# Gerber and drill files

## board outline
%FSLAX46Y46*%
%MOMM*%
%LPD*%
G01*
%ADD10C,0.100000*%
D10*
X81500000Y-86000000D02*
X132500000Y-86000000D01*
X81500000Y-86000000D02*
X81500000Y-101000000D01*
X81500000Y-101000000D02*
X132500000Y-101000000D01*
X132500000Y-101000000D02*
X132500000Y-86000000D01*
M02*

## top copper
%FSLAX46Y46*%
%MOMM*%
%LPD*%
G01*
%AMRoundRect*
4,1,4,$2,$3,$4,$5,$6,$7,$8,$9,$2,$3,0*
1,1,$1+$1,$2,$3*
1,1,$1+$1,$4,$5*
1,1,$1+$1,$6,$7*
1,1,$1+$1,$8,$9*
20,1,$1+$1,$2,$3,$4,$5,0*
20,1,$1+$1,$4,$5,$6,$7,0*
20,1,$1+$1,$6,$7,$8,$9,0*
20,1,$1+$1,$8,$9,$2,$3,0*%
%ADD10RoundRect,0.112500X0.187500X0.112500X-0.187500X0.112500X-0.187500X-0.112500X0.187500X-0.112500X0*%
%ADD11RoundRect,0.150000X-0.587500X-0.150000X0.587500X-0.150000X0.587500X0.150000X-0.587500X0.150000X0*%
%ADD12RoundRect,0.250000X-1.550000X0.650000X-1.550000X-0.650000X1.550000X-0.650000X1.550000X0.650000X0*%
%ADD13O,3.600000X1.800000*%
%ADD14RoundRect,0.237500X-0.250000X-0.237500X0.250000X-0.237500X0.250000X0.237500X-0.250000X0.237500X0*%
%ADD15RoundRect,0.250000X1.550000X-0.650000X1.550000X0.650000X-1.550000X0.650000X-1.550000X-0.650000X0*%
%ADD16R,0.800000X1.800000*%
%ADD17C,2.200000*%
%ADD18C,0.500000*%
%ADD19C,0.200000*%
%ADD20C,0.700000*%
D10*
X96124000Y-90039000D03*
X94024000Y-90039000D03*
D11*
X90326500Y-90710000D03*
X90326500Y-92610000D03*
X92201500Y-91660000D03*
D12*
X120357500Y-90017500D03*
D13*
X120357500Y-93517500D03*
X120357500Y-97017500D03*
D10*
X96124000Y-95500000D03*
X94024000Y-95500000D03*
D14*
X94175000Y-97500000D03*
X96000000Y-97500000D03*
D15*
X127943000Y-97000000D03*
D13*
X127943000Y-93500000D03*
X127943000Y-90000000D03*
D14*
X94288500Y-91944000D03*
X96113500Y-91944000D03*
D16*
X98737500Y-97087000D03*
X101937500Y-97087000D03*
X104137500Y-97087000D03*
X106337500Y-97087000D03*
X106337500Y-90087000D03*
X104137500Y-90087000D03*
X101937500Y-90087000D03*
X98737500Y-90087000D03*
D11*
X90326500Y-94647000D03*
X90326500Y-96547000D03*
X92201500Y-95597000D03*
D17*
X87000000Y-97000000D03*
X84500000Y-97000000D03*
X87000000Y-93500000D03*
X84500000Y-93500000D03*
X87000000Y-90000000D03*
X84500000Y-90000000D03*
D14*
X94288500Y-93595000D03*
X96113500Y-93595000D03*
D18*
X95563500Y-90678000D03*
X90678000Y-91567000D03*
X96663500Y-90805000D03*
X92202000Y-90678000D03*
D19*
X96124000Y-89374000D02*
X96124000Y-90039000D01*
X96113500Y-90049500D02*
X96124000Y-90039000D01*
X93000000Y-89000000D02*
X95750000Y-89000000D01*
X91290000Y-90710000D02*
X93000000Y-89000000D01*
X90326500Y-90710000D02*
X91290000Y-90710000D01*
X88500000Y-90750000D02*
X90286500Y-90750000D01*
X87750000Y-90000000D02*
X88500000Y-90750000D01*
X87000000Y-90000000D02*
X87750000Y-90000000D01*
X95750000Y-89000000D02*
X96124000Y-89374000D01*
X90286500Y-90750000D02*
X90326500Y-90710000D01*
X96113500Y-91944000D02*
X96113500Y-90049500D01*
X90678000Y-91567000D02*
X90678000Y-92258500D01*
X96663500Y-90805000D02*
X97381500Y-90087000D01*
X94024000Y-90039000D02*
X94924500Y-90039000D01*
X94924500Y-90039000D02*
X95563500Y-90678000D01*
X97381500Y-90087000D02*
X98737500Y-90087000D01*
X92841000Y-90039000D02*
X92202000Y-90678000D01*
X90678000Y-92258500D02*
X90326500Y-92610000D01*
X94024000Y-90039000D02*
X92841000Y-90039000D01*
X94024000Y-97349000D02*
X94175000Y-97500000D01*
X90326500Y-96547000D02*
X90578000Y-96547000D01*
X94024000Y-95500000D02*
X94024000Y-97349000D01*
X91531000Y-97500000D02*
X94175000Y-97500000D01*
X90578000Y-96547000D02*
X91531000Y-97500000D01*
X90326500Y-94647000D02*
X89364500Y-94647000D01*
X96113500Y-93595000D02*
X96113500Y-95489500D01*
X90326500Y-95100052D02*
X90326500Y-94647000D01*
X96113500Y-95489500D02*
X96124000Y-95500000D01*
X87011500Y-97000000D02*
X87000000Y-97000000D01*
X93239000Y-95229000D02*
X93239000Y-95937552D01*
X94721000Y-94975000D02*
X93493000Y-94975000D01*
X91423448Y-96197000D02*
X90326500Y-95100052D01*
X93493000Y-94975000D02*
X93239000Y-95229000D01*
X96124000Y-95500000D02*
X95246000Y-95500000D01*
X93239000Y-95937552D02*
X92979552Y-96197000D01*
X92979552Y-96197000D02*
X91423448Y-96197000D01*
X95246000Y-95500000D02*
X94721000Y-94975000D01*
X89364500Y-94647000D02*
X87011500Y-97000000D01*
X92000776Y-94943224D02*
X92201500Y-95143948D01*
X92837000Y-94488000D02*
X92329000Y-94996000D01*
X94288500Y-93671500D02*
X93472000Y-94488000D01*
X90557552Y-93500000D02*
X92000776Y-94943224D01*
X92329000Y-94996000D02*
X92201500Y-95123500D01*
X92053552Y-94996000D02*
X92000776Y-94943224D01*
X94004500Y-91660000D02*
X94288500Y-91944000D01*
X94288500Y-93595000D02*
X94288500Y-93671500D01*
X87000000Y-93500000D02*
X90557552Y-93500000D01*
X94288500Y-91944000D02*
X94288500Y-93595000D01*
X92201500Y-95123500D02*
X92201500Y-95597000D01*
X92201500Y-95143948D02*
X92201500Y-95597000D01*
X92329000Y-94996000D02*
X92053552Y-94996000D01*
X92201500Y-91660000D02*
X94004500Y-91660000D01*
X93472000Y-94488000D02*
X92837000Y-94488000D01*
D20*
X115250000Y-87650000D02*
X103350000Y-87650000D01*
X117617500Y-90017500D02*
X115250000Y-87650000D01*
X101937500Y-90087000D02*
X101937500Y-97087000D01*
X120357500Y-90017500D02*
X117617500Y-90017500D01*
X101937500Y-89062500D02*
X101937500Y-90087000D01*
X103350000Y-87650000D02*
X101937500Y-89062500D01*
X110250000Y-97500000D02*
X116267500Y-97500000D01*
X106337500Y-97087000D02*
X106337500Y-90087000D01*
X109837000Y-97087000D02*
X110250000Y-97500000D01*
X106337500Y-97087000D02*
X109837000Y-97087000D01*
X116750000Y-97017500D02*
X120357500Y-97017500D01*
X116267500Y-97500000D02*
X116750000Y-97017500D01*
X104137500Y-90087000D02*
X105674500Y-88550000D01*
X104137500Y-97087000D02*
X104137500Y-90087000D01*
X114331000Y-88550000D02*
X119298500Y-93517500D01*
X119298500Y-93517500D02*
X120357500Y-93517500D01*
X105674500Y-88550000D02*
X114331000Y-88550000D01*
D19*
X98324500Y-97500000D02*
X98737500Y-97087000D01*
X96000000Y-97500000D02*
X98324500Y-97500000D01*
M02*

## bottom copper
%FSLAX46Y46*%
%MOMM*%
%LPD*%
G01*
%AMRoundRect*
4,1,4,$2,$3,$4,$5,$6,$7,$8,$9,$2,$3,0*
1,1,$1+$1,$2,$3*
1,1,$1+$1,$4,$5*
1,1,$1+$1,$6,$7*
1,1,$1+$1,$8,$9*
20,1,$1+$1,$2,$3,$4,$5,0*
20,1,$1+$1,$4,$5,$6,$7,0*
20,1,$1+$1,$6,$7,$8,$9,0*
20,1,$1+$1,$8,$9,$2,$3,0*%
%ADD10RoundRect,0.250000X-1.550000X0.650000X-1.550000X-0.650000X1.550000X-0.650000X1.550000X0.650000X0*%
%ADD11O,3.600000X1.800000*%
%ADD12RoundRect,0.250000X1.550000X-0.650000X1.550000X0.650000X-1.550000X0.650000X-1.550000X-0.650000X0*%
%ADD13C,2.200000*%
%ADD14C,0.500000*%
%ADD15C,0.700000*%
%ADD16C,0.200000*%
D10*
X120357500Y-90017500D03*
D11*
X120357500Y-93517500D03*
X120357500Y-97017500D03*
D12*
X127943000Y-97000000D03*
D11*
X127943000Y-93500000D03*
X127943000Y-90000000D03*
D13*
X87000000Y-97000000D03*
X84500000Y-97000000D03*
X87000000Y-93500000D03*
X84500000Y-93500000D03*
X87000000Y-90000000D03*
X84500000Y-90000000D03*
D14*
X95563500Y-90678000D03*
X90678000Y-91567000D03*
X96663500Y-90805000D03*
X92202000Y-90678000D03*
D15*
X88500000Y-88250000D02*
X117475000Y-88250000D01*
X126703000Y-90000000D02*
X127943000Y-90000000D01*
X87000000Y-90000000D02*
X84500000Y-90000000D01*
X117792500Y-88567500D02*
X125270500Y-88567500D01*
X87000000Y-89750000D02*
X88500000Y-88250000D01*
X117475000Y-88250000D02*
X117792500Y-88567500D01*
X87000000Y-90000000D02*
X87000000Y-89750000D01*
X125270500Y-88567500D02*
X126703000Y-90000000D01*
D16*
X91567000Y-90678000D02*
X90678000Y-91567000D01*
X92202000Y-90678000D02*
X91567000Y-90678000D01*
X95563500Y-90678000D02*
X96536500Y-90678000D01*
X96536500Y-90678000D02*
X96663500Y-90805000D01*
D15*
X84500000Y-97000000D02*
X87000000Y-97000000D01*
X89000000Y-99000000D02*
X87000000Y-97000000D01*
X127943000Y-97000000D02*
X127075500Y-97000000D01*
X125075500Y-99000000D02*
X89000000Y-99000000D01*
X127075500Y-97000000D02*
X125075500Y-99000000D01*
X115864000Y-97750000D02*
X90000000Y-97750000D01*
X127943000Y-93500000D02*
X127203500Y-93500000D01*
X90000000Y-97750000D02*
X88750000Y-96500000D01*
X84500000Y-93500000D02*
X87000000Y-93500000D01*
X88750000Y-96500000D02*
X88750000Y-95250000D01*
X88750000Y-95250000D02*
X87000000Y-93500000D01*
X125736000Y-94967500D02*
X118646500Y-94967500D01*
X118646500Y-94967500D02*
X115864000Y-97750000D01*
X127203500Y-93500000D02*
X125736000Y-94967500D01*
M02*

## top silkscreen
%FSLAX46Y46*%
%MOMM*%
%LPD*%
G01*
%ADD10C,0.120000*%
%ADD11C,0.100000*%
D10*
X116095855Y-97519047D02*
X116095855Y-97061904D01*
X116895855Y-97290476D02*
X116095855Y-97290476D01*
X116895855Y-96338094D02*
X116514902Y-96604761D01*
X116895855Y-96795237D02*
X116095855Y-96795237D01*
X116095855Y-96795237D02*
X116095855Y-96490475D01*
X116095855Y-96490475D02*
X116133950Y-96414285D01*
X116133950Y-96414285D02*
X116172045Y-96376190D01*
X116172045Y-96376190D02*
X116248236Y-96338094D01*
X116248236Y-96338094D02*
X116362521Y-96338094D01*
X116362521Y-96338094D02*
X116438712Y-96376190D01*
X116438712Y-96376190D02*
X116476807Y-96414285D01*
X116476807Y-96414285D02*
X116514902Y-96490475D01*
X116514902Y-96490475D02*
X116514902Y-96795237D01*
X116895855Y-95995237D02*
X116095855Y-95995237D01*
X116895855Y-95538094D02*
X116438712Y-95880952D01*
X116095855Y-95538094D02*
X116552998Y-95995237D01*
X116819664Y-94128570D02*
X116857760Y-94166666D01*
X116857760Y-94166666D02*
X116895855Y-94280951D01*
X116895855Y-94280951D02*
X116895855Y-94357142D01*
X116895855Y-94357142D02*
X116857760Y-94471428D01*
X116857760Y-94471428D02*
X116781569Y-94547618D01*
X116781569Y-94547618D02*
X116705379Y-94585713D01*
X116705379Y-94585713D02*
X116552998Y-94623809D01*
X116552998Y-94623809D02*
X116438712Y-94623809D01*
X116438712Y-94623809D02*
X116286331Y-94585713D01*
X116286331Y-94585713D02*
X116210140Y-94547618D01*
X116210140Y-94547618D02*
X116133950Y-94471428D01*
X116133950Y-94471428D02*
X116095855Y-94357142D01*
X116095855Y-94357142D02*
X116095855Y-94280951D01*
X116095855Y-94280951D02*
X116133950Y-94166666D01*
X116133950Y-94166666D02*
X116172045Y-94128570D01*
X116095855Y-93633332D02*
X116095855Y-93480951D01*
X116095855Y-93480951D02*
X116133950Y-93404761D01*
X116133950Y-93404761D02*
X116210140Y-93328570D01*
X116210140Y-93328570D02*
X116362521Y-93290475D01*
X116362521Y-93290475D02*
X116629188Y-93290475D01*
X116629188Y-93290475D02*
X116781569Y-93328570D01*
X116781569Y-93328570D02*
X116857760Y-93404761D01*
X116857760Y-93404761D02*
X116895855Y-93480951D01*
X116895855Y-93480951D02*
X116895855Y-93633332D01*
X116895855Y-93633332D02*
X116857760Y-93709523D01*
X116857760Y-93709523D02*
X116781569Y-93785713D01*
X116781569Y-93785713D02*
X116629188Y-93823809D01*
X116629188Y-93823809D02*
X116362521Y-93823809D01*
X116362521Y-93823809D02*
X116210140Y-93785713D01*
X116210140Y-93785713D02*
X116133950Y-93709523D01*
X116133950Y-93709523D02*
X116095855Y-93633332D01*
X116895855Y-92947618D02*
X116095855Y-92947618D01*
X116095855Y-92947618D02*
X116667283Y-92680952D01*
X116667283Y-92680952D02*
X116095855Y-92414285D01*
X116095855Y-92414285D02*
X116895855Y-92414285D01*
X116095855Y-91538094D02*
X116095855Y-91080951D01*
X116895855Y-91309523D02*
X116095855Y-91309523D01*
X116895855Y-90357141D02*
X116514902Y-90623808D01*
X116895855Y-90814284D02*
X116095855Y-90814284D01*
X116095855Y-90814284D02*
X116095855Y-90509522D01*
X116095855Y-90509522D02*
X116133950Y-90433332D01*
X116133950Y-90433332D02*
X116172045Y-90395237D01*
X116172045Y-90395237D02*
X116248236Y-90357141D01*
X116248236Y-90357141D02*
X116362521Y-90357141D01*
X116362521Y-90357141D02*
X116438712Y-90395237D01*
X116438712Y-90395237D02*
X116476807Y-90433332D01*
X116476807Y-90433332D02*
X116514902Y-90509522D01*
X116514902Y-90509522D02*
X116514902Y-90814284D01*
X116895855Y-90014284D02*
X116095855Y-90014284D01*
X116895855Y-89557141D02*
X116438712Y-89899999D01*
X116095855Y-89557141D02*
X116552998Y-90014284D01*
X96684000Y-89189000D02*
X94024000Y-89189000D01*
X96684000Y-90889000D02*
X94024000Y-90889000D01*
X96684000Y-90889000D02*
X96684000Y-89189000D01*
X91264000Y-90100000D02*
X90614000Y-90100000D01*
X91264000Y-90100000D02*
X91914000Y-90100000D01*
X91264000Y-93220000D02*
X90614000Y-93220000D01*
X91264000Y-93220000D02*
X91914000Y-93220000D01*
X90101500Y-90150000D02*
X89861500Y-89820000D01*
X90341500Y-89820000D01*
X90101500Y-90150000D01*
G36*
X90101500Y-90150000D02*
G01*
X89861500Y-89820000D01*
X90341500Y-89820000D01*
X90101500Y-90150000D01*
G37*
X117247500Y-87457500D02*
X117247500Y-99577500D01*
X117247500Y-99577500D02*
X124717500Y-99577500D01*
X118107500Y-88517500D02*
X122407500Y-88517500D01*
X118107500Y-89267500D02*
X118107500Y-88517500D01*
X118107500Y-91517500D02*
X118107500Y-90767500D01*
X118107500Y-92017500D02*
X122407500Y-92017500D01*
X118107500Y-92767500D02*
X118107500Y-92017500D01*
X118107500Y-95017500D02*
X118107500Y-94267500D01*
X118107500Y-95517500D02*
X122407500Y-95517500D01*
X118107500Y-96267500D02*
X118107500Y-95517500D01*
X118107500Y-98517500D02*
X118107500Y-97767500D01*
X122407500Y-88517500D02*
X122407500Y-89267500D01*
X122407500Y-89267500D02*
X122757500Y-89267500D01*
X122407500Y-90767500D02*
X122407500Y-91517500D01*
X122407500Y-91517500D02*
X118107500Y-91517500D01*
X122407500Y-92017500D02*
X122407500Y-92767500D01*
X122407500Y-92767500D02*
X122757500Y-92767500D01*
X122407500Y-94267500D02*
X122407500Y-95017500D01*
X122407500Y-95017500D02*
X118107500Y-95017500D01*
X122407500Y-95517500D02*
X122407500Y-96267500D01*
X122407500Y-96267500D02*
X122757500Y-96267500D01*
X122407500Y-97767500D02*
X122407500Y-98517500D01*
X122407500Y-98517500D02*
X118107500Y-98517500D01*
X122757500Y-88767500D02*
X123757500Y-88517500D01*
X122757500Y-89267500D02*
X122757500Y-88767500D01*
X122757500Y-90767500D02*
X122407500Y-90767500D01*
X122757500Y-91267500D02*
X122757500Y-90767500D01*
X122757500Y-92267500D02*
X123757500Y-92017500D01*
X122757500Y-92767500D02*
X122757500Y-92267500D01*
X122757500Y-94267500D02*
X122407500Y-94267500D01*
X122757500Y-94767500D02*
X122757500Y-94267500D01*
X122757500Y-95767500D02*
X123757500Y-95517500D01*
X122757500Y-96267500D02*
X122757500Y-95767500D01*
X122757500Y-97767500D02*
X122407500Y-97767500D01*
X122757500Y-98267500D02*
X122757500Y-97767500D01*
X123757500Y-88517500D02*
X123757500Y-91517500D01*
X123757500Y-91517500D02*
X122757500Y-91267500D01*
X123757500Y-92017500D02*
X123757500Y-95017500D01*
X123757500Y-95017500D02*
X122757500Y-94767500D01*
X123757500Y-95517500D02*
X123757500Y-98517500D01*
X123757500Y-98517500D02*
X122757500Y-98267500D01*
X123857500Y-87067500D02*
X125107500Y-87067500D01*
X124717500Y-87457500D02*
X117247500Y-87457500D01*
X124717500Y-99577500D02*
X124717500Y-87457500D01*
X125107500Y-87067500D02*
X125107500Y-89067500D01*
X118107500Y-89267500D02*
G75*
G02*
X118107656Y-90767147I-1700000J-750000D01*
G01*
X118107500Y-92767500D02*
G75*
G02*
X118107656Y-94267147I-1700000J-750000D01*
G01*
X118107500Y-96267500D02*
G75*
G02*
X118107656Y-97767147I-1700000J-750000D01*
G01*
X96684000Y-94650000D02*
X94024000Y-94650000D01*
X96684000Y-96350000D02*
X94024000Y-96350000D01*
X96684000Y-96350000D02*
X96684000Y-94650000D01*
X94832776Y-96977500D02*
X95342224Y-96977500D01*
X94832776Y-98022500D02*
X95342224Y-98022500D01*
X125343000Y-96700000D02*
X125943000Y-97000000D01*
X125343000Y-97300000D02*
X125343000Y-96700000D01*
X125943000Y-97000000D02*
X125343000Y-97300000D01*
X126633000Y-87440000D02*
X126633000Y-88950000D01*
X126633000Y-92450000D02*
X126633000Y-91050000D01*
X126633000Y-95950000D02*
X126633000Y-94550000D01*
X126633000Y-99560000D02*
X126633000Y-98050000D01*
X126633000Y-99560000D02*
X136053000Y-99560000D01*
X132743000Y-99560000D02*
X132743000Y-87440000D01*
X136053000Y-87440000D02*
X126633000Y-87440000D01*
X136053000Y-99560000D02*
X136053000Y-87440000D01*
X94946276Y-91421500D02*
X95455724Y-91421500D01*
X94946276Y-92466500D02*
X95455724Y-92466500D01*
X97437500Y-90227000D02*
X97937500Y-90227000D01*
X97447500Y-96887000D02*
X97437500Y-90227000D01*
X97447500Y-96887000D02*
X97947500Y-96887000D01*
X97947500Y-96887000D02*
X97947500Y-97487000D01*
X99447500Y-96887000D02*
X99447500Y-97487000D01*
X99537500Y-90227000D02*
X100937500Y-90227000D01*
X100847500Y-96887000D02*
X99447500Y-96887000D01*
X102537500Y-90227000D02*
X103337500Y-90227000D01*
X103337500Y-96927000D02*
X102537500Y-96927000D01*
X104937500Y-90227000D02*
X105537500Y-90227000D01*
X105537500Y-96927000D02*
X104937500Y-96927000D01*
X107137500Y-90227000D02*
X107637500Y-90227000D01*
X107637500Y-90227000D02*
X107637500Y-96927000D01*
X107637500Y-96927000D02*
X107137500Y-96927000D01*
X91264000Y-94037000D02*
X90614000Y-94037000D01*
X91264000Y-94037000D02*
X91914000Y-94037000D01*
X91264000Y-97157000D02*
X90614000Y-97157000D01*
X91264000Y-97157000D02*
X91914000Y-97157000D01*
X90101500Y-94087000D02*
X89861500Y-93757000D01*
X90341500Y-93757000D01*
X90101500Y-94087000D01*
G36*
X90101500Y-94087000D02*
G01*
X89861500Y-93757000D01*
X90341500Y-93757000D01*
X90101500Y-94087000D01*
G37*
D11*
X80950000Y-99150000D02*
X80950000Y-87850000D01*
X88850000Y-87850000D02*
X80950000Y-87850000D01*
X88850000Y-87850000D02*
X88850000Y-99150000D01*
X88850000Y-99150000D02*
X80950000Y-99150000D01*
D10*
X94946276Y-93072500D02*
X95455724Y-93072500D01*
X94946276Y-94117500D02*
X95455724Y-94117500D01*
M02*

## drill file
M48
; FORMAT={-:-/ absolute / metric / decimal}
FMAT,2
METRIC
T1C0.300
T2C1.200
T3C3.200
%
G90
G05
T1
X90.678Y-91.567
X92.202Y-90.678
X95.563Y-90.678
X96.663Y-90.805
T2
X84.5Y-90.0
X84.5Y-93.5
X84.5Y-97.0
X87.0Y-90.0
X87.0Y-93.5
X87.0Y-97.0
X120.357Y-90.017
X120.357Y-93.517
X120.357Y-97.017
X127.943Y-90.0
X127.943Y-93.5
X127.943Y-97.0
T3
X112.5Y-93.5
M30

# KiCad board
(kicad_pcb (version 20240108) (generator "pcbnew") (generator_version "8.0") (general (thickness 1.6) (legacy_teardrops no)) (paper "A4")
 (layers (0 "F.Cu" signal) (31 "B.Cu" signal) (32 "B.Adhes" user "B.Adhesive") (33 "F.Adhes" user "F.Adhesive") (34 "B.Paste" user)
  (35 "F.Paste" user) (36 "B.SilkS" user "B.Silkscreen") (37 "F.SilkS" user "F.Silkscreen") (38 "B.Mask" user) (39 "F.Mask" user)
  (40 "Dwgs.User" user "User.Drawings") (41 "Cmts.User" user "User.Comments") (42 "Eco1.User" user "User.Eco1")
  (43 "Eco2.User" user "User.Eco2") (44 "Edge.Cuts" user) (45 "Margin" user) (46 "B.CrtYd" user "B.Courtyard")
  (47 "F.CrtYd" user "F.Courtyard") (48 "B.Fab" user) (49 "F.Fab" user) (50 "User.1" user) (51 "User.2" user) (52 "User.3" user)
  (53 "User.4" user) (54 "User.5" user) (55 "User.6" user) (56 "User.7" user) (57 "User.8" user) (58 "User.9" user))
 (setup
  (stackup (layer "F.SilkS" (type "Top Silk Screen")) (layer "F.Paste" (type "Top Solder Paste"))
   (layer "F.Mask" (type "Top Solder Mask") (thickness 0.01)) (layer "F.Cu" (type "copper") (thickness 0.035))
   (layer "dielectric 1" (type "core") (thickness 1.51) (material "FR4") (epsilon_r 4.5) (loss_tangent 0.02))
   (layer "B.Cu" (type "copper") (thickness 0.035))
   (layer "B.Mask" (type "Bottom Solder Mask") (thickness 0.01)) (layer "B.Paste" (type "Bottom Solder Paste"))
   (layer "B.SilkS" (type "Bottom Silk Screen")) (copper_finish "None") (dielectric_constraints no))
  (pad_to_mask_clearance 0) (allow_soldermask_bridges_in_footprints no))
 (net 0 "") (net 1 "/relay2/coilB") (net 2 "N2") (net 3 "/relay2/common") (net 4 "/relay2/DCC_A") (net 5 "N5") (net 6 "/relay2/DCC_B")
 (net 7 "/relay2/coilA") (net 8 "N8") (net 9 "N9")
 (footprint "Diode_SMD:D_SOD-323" (layer "F.Cu") (at 95.074 90.039 180)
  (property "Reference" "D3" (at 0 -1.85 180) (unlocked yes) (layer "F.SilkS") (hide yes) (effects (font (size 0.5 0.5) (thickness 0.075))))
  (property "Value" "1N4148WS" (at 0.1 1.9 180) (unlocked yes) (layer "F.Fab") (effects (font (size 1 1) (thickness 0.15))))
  (fp_line (start -1.61 0.85) (end 1.05 0.85) (stroke (width 0.12) (type solid)) (layer "F.SilkS"))
  (fp_line (start -1.61 -0.85) (end 1.05 -0.85) (stroke (width 0.12) (type solid)) (layer "F.SilkS"))
  (fp_line (start -1.61 -0.85) (end -1.61 0.85) (stroke (width 0.12) (type solid)) (layer "F.SilkS"))
  (pad "1" smd roundrect (at -1.05 0 180) (size 0.6 0.45) (layers "F.Cu" "F.Paste" "F.Mask") (roundrect_rratio 0.25) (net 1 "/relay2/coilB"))
  (pad "2" smd roundrect (at 1.05 0 180) (size 0.6 0.45) (layers "F.Cu" "F.Paste" "F.Mask") (roundrect_rratio 0.25) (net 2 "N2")))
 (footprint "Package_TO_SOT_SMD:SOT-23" (layer "F.Cu") (at 91.264 91.66)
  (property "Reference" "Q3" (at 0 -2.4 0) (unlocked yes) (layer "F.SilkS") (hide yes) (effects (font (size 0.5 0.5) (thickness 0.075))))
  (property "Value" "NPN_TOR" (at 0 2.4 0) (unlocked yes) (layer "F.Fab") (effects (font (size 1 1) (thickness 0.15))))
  (fp_line (start 0 -1.56) (end -0.65 -1.56) (stroke (width 0.12) (type solid)) (layer "F.SilkS"))
  (fp_line (start 0 -1.56) (end 0.65 -1.56) (stroke (width 0.12) (type solid)) (layer "F.SilkS"))
  (fp_line (start 0 1.56) (end -0.65 1.56) (stroke (width 0.12) (type solid)) (layer "F.SilkS"))
  (fp_line (start 0 1.56) (end 0.65 1.56) (stroke (width 0.12) (type solid)) (layer "F.SilkS"))
  (fp_poly
   (pts (xy -1.1625 -1.51) (xy -1.4025 -1.84) (xy -0.9225 -1.84) (xy -1.1625 -1.51)) (stroke (width 0.12) (type solid)) (fill solid)
   (layer "F.SilkS"))
  (pad "1" smd roundrect (at -0.9375 -0.95) (size 1.475 0.6) (layers "F.Cu" "F.Paste" "F.Mask") (roundrect_rratio 0.25)
   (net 1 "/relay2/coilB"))
  (pad "2" smd roundrect (at -0.9375 0.95) (size 1.475 0.6) (layers "F.Cu" "F.Paste" "F.Mask") (roundrect_rratio 0.25) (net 2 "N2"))
  (pad "3" smd roundrect (at 0.9375 0) (size 1.475 0.6) (layers "F.Cu" "F.Paste" "F.Mask") (roundrect_rratio 0.25) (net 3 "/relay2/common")))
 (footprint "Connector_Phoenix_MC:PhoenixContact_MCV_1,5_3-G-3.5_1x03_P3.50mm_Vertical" (layer "F.Cu") (at 120.3575 90.0175 -90)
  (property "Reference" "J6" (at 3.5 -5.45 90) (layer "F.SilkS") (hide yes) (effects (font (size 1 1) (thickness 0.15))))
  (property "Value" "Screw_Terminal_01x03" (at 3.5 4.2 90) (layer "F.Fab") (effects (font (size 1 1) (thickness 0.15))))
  (fp_line (start -2.56 3.11) (end 9.56 3.11) (stroke (width 0.12) (type solid)) (layer "F.SilkS"))
  (fp_line (start 9.56 3.11) (end 9.56 -4.36) (stroke (width 0.12) (type solid)) (layer "F.SilkS"))
  (fp_line (start -1.5 2.25) (end -1.5 -2.05) (stroke (width 0.12) (type solid)) (layer "F.SilkS"))
  (fp_line (start -0.75 2.25) (end -1.5 2.25) (stroke (width 0.12) (type solid)) (layer "F.SilkS"))
  (fp_line (start 1.5 2.25) (end 0.75 2.25) (stroke (width 0.12) (type solid)) (layer "F.SilkS"))
  (fp_line (start 2 2.25) (end 2 -2.05) (stroke (width 0.12) (type solid)) (layer "F.SilkS"))
  (fp_line (start 2.75 2.25) (end 2 2.25) (stroke (width 0.12) (type solid)) (layer "F.SilkS"))
  (fp_line (start 5 2.25) (end 4.25 2.25) (stroke (width 0.12) (type solid)) (layer "F.SilkS"))
  (fp_line (start 5.5 2.25) (end 5.5 -2.05) (stroke (width 0.12) (type solid)) (layer "F.SilkS"))
  (fp_line (start 6.25 2.25) (end 5.5 2.25) (stroke (width 0.12) (type solid)) (layer "F.SilkS"))
  (fp_line (start 8.5 2.25) (end 7.75 2.25) (stroke (width 0.12) (type solid)) (layer "F.SilkS"))
  (fp_line (start -1.5 -2.05) (end -0.75 -2.05) (stroke (width 0.12) (type solid)) (layer "F.SilkS"))
  (fp_line (start -0.75 -2.05) (end -0.75 -2.4) (stroke (width 0.12) (type solid)) (layer "F.SilkS"))
  (fp_line (start 0.75 -2.05) (end 1.5 -2.05) (stroke (width 0.12) (type solid)) (layer "F.SilkS"))
  (fp_line (start 1.5 -2.05) (end 1.5 2.25) (stroke (width 0.12) (type solid)) (layer "F.SilkS"))
  (fp_line (start 2 -2.05) (end 2.75 -2.05) (stroke (width 0.12) (type solid)) (layer "F.SilkS"))
  (fp_line (start 2.75 -2.05) (end 2.75 -2.4) (stroke (width 0.12) (type solid)) (layer "F.SilkS"))
  (fp_line (start 4.25 -2.05) (end 5 -2.05) (stroke (width 0.12) (type solid)) (layer "F.SilkS"))
  (fp_line (start 5 -2.05) (end 5 2.25) (stroke (width 0.12) (type solid)) (layer "F.SilkS"))
  (fp_line (start 5.5 -2.05) (end 6.25 -2.05) (stroke (width 0.12) (type solid)) (layer "F.SilkS"))
  (fp_line (start 6.25 -2.05) (end 6.25 -2.4) (stroke (width 0.12) (type solid)) (layer "F.SilkS"))
  (fp_line (start 7.75 -2.05) (end 8.5 -2.05) (stroke (width 0.12) (type solid)) (layer "F.SilkS"))
  (fp_line (start 8.5 -2.05) (end 8.5 2.25) (stroke (width 0.12) (type solid)) (layer "F.SilkS"))
  (fp_line (start -1.25 -2.4) (end -1.5 -3.4) (stroke (width 0.12) (type solid)) (layer "F.SilkS"))
  (fp_line (start -0.75 -2.4) (end -1.25 -2.4) (stroke (width 0.12) (type solid)) (layer "F.SilkS"))
  (fp_line (start 0.75 -2.4) (end 0.75 -2.05) (stroke (width 0.12) (type solid)) (layer "F.SilkS"))
  (fp_line (start 1.25 -2.4) (end 0.75 -2.4) (stroke (width 0.12) (type solid)) (layer "F.SilkS"))
  (fp_line (start 2.25 -2.4) (end 2 -3.4) (stroke (width 0.12) (type solid)) (layer "F.SilkS"))
  (fp_line (start 2.75 -2.4) (end 2.25 -2.4) (stroke (width 0.12) (type solid)) (layer "F.SilkS"))
  (fp_line (start 4.25 -2.4) (end 4.25 -2.05) (stroke (width 0.12) (type solid)) (layer "F.SilkS"))
  (fp_line (start 4.75 -2.4) (end 4.25 -2.4) (stroke (width 0.12) (type solid)) (layer "F.SilkS"))
  (fp_line (start 5.75 -2.4) (end 5.5 -3.4) (stroke (width 0.12) (type solid)) (layer "F.SilkS"))
  (fp_line (start 6.25 -2.4) (end 5.75 -2.4) (stroke (width 0.12) (type solid)) (layer "F.SilkS"))
  (fp_line (start 7.75 -2.4) (end 7.75 -2.05) (stroke (width 0.12) (type solid)) (layer "F.SilkS"))
  (fp_line (start 8.25 -2.4) (end 7.75 -2.4) (stroke (width 0.12) (type solid)) (layer "F.SilkS"))
  (fp_line (start -1.5 -3.4) (end 1.5 -3.4) (stroke (width 0.12) (type solid)) (layer "F.SilkS"))
  (fp_line (start 1.5 -3.4) (end 1.25 -2.4) (stroke (width 0.12) (type solid)) (layer "F.SilkS"))
  (fp_line (start 2 -3.4) (end 5 -3.4) (stroke (width 0.12) (type solid)) (layer "F.SilkS"))
  (fp_line (start 5 -3.4) (end 4.75 -2.4) (stroke (width 0.12) (type solid)) (layer "F.SilkS"))
  (fp_line (start 5.5 -3.4) (end 8.5 -3.4) (stroke (width 0.12) (type solid)) (layer "F.SilkS"))
  (fp_line (start 8.5 -3.4) (end 8.25 -2.4) (stroke (width 0.12) (type solid)) (layer "F.SilkS"))
  (fp_line (start -2.95 -3.5) (end -2.95 -4.75) (stroke (width 0.12) (type solid)) (layer "F.SilkS"))
  (fp_line (start -2.56 -4.36) (end -2.56 3.11) (stroke (width 0.12) (type solid)) (layer "F.SilkS"))
  (fp_line (start 9.56 -4.36) (end -2.56 -4.36) (stroke (width 0.12) (type solid)) (layer "F.SilkS"))
  (fp_line (start -2.95 -4.75) (end -0.95 -4.75) (stroke (width 0.12) (type solid)) (layer "F.SilkS"))
  (fp_arc (start -0.75 2.25) (mid -0.000193 2.09191) (end 0.749647 2.249844) (stroke (width 0.12) (type solid)) (layer "F.SilkS"))
  (fp_arc (start 2.75 2.25) (mid 3.499807 2.09191) (end 4.249647 2.249844) (stroke (width 0.12) (type solid)) (layer "F.SilkS"))
  (fp_arc (start 6.25 2.25) (mid 6.999807 2.09191) (end 7.749647 2.249844) (stroke (width 0.12) (type solid)) (layer "F.SilkS"))
  (pad "1" thru_hole roundrect (at 0 0 270) (size 1.8 3.6) (drill 1.2) (layers "*.Cu" "*.Mask") (remove_unused_layers no)
   (roundrect_rratio 0.138889) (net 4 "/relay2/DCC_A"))
  (pad "2" thru_hole oval (at 3.5 0 270) (size 1.8 3.6) (drill 1.2) (layers "*.Cu" "*.Mask") (remove_unused_layers no) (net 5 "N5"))
  (pad "3" thru_hole oval (at 7 0 270) (size 1.8 3.6) (drill 1.2) (layers "*.Cu" "*.Mask") (remove_unused_layers no) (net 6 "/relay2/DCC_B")))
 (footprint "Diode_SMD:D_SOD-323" (layer "F.Cu") (at 95.074 95.5 180)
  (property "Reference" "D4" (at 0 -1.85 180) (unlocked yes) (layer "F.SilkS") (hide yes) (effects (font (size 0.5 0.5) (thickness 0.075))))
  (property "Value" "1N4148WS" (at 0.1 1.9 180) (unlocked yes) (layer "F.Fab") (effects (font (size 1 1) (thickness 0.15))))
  (fp_line (start -1.61 0.85) (end 1.05 0.85) (stroke (width 0.12) (type solid)) (layer "F.SilkS"))
  (fp_line (start -1.61 -0.85) (end 1.05 -0.85) (stroke (width 0.12) (type solid)) (layer "F.SilkS"))
  (fp_line (start -1.61 -0.85) (end -1.61 0.85) (stroke (width 0.12) (type solid)) (layer "F.SilkS"))
  (pad "1" smd roundrect (at -1.05 0 180) (size 0.6 0.45) (layers "F.Cu" "F.Paste" "F.Mask") (roundrect_rratio 0.25) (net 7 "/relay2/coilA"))
  (pad "2" smd roundrect (at 1.05 0 180) (size 0.6 0.45) (layers "F.Cu" "F.Paste" "F.Mask") (roundrect_rratio 0.25) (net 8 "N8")))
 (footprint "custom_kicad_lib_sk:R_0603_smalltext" (layer "F.Cu") (at 95.0875 97.5)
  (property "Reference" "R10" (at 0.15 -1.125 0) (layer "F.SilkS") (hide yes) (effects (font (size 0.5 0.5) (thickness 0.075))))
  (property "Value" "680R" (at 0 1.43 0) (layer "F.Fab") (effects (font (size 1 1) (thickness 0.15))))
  (fp_line (start -0.254724 -0.5225) (end 0.254724 -0.5225) (stroke (width 0.12) (type solid)) (layer "F.SilkS"))
  (fp_line (start -0.254724 0.5225) (end 0.254724 0.5225) (stroke (width 0.12) (type solid)) (layer "F.SilkS"))
  (pad "1" smd roundrect (at -0.9125 0) (size 0.975 0.95) (layers "F.Cu" "F.Paste" "F.Mask") (roundrect_rratio 0.25) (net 8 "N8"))
  (pad "2" smd roundrect (at 0.9125 0) (size 0.975 0.95) (layers "F.Cu" "F.Paste" "F.Mask") (roundrect_rratio 0.25) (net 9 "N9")))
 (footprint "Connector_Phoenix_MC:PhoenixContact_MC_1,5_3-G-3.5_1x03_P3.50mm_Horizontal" (layer "F.Cu") (at 127.943 97 90)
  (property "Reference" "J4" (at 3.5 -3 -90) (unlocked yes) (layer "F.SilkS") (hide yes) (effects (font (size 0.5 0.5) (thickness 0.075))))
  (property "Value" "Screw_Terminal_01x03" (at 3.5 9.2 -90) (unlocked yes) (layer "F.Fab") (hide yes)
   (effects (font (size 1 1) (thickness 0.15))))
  (fp_line (start 0.3 -2.6) (end 0 -2) (stroke (width 0.12) (type solid)) (layer "F.SilkS"))
  (fp_line (start -0.3 -2.6) (end 0.3 -2.6) (stroke (width 0.12) (type solid)) (layer "F.SilkS"))
  (fp_line (start 0 -2) (end -0.3 -2.6) (stroke (width 0.12) (type solid)) (layer "F.SilkS"))
  (fp_line (start 9.56 -1.31) (end 8.05 -1.31) (stroke (width 0.12) (type solid)) (layer "F.SilkS"))
  (fp_line (start 4.55 -1.31) (end 5.95 -1.31) (stroke (width 0.12) (type solid)) (layer "F.SilkS"))
  (fp_line (start 1.05 -1.31) (end 2.45 -1.31) (stroke (width 0.12) (type solid)) (layer "F.SilkS"))
  (fp_line (start -2.56 -1.31) (end -1.05 -1.31) (stroke (width 0.12) (type solid)) (layer "F.SilkS"))
  (fp_line (start -2.56 -1.31) (end -2.56 8.11) (stroke (width 0.12) (type solid)) (layer "F.SilkS"))
  (fp_line (start -2.56 4.8) (end 9.56 4.8) (stroke (width 0.12) (type solid)) (layer "F.SilkS"))
  (fp_line (start 9.56 8.11) (end 9.56 -1.31) (stroke (width 0.12) (type solid)) (layer "F.SilkS"))
  (fp_line (start -2.56 8.11) (end 9.56 8.11) (stroke (width 0.12) (type solid)) (layer "F.SilkS"))
  (pad "1" thru_hole roundrect (at 0 0 90) (size 1.8 3.6) (drill 1.2) (layers "*.Cu" "*.Mask") (remove_unused_layers no)
   (roundrect_rratio 0.138889) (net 7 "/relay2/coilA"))
  (pad "2" thru_hole oval (at 3.5 0 90) (size 1.8 3.6) (drill 1.2) (layers "*.Cu" "*.Mask") (remove_unused_layers no)
   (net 3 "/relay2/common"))
  (pad "3" thru_hole oval (at 7 0 90) (size 1.8 3.6) (drill 1.2) (layers "*.Cu" "*.Mask") (remove_unused_layers no) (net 1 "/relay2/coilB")))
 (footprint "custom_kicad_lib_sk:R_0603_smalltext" (layer "F.Cu") (at 95.201 91.944)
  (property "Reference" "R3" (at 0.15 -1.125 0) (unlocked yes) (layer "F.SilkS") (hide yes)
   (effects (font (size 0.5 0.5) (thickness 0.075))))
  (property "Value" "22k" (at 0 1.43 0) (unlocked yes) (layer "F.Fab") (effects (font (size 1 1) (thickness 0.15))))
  (fp_line (start -0.254724 -0.5225) (end 0.254724 -0.5225) (stroke (width 0.12) (type solid)) (layer "F.SilkS"))
  (fp_line (start -0.254724 0.5225) (end 0.254724 0.5225) (stroke (width 0.12) (type solid)) (layer "F.SilkS"))
  (pad "1" smd roundrect (at -0.9125 0) (size 0.975 0.95) (layers "F.Cu" "F.Paste" "F.Mask") (roundrect_rratio 0.25)
   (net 3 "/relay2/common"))
  (pad "2" smd roundrect (at 0.9125 0) (size 0.975 0.95) (layers "F.Cu" "F.Paste" "F.Mask") (roundrect_rratio 0.25) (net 1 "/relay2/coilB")))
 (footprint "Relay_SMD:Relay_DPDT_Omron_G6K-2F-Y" (layer "F.Cu") (at 102.5375 93.587 90)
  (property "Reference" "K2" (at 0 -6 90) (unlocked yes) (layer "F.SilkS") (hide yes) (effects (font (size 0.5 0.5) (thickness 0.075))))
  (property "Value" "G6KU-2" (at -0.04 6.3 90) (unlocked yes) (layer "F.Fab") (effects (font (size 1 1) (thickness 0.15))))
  (fp_line (start 3.36 -5.1) (end 3.36 -4.6) (stroke (width 0.12) (type solid)) (layer "F.SilkS"))
  (fp_line (start -3.3 -5.09) (end 3.36 -5.1) (stroke (width 0.12) (type solid)) (layer "F.SilkS"))
  (fp_line (start -3.3 -5.09) (end -3.3 -4.59) (stroke (width 0.12) (type solid)) (layer "F.SilkS"))
  (fp_line (start -3.3 -4.59) (end -3.9 -4.59) (stroke (width 0.12) (type solid)) (layer "F.SilkS"))
  (fp_line (start -3.3 -3.09) (end -3.9 -3.09) (stroke (width 0.12) (type solid)) (layer "F.SilkS"))
  (fp_line (start 3.36 -3) (end 3.36 -1.6) (stroke (width 0.12) (type solid)) (layer "F.SilkS"))
  (fp_line (start -3.3 -1.69) (end -3.3 -3.09) (stroke (width 0.12) (type solid)) (layer "F.SilkS"))
  (fp_line (start 3.36 0) (end 3.36 0.8) (stroke (width 0.12) (type solid)) (layer "F.SilkS"))
  (fp_line (start -3.34 0.8) (end -3.34 0) (stroke (width 0.12) (type solid)) (layer "F.SilkS"))
  (fp_line (start 3.36 2.4) (end 3.36 3) (stroke (width 0.12) (type solid)) (layer "F.SilkS"))
  (fp_line (start -3.34 3) (end -3.34 2.4) (stroke (width 0.12) (type solid)) (layer "F.SilkS"))
  (fp_line (start 3.36 4.6) (end 3.36 5.1) (stroke (width 0.12) (type solid)) (layer "F.SilkS"))
  (fp_line (start 3.36 5.1) (end -3.34 5.1) (stroke (width 0.12) (type solid)) (layer "F.SilkS"))
  (fp_line (start -3.34 5.1) (end -3.34 4.6) (stroke (width 0.12) (type solid)) (layer "F.SilkS"))
  (pad "1" smd rect (at -3.5 -3.8 90) (size 1.8 0.8) (layers "F.Cu" "F.Paste" "F.Mask") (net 9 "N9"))
  (pad "2" smd rect (at -3.5 -0.6 90) (size 1.8 0.8) (layers "F.Cu" "F.Paste" "F.Mask") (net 4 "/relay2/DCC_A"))
  (pad "3" smd rect (at -3.5 1.6 90) (size 1.8 0.8) (layers "F.Cu" "F.Paste" "F.Mask") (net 5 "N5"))
  (pad "4" smd rect (at -3.5 3.8 90) (size 1.8 0.8) (layers "F.Cu" "F.Paste" "F.Mask") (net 6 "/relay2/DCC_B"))
  (pad "5" smd rect (at 3.5 3.8 90) (size 1.8 0.8) (layers "F.Cu" "F.Paste" "F.Mask") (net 6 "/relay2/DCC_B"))
  (pad "6" smd rect (at 3.5 1.6 90) (size 1.8 0.8) (layers "F.Cu" "F.Paste" "F.Mask") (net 5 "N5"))
  (pad "7" smd rect (at 3.5 -0.6 90) (size 1.8 0.8) (layers "F.Cu" "F.Paste" "F.Mask") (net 4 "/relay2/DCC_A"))
  (pad "8" smd rect (at 3.5 -3.8 90) (size 1.8 0.8) (layers "F.Cu" "F.Paste" "F.Mask") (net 2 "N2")))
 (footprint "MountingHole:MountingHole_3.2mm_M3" (layer "F.Cu") (at 112.5 93.5)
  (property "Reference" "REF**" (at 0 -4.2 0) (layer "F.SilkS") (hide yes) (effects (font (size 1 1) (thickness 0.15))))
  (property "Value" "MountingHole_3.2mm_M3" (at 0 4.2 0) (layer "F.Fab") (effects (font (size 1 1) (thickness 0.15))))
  (pad "" np_thru_hole circle (at 0 0) (size 3.2 3.2) (drill 3.2) (layers "*.Cu" "*.Mask")))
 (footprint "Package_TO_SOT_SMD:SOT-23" (layer "F.Cu") (at 91.264 95.597)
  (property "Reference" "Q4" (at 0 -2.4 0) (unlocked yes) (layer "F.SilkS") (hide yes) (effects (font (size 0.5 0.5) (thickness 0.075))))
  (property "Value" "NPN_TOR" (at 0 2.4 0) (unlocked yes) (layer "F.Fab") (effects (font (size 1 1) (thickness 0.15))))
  (fp_line (start 0 -1.56) (end -0.65 -1.56) (stroke (width 0.12) (type solid)) (layer "F.SilkS"))
  (fp_line (start 0 -1.56) (end 0.65 -1.56) (stroke (width 0.12) (type solid)) (layer "F.SilkS"))
  (fp_line (start 0 1.56) (end -0.65 1.56) (stroke (width 0.12) (type solid)) (layer "F.SilkS"))
  (fp_line (start 0 1.56) (end 0.65 1.56) (stroke (width 0.12) (type solid)) (layer "F.SilkS"))
  (fp_poly
   (pts (xy -1.1625 -1.51) (xy -1.4025 -1.84) (xy -0.9225 -1.84) (xy -1.1625 -1.51)) (stroke (width 0.12) (type solid)) (fill solid)
   (layer "F.SilkS"))
  (pad "1" smd roundrect (at -0.9375 -0.95) (size 1.475 0.6) (layers "F.Cu" "F.Paste" "F.Mask") (roundrect_rratio 0.25)
   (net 7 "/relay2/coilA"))
  (pad "2" smd roundrect (at -0.9375 0.95) (size 1.475 0.6) (layers "F.Cu" "F.Paste" "F.Mask") (roundrect_rratio 0.25) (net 8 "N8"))
  (pad "3" smd roundrect (at 0.9375 0) (size 1.475 0.6) (layers "F.Cu" "F.Paste" "F.Mask") (roundrect_rratio 0.25) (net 3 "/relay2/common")))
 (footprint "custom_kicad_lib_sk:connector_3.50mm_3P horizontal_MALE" (layer "F.Cu") (at 87 93.5 -90)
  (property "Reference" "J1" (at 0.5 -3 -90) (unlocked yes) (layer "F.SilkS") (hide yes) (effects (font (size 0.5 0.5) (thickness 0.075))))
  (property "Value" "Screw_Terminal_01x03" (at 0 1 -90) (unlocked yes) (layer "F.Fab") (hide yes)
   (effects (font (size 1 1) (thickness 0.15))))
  (fp_line (start 5.65 6.05) (end -5.65 6.05) (stroke (width 0.1) (type default)) (layer "F.SilkS"))
  (fp_line (start -5.65 -1.85) (end -5.65 6.05) (stroke (width 0.1) (type default)) (layer "F.SilkS"))
  (fp_line (start -5.65 -1.85) (end 5.65 -1.85) (stroke (width 0.1) (type default)) (layer "F.SilkS"))
  (fp_line (start 5.65 -1.85) (end 5.65 6.05) (stroke (width 0.1) (type default)) (layer "F.SilkS"))
  (pad "1" thru_hole circle (at 3.5 0 270) (size 2.2 2.2) (drill 1.2) (layers "*.Cu" "*.Mask") (remove_unused_layers no)
   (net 7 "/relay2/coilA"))
  (pad "1" thru_hole circle (at 3.5 2.5 270) (size 2.2 2.2) (drill 1.2) (layers "*.Cu" "*.Mask") (remove_unused_layers no)
   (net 7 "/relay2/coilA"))
  (pad "2" thru_hole circle (at 0 0 270) (size 2.2 2.2) (drill 1.2) (layers "*.Cu" "*.Mask") (remove_unused_layers no)
   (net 3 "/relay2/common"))
  (pad "2" thru_hole circle (at 0 2.5 270) (size 2.2 2.2) (drill 1.2) (layers "*.Cu" "*.Mask") (remove_unused_layers no)
   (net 3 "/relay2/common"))
  (pad "3" thru_hole circle (at -3.5 0 270) (size 2.2 2.2) (drill 1.2) (layers "*.Cu" "*.Mask") (remove_unused_layers no)
   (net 1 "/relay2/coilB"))
  (pad "3" thru_hole circle (at -3.5 2.5 270) (size 2.2 2.2) (drill 1.2) (layers "*.Cu" "*.Mask") (remove_unused_layers no)
   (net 1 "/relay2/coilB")))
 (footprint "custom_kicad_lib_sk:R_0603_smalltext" (layer "F.Cu") (at 95.201 93.595)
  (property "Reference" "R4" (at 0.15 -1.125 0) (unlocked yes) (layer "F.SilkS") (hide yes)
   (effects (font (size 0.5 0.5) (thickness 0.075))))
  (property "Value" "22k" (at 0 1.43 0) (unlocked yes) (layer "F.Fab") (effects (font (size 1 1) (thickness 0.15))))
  (fp_line (start -0.254724 -0.5225) (end 0.254724 -0.5225) (stroke (width 0.12) (type solid)) (layer "F.SilkS"))
  (fp_line (start -0.254724 0.5225) (end 0.254724 0.5225) (stroke (width 0.12) (type solid)) (layer "F.SilkS"))
  (pad "1" smd roundrect (at -0.9125 0) (size 0.975 0.95) (layers "F.Cu" "F.Paste" "F.Mask") (roundrect_rratio 0.25)
   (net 3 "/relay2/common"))
  (pad "2" smd roundrect (at 0.9125 0) (size 0.975 0.95) (layers "F.Cu" "F.Paste" "F.Mask") (roundrect_rratio 0.25) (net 7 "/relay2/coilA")))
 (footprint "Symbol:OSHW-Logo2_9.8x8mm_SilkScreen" (layer "B.Cu") (at 100.5 93.5 -90)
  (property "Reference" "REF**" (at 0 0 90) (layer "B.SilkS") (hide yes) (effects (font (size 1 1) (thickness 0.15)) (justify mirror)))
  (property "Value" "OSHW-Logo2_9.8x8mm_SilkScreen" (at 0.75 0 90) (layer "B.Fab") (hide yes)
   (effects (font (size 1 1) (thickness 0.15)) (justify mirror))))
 (gr_line (start 81.5 86) (end 132.5 86) (stroke (width 0.1) (type default)) (layer "Edge.Cuts"))
 (gr_line (start 81.5 86) (end 81.5 101) (stroke (width 0.1) (type default)) (layer "Edge.Cuts"))
 (gr_line (start 81.5 101) (end 132.5 101) (stroke (width 0.1) (type default)) (layer "Edge.Cuts"))
 (gr_line (start 132.5 101) (end 132.5 86) (stroke (width 0.1) (type default)) (layer "Edge.Cuts"))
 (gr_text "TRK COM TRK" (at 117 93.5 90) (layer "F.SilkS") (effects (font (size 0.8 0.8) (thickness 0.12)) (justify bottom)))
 (segment (start 96.124 89.374) (end 96.124 90.039) (width 0.2) (layer "F.Cu") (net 1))
 (segment (start 96.1135 90.0495) (end 96.124 90.039) (width 0.2) (layer "F.Cu") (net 1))
 (segment (start 93 89) (end 95.75 89) (width 0.2) (layer "F.Cu") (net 1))
 (segment (start 91.29 90.71) (end 93 89) (width 0.2) (layer "F.Cu") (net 1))
 (segment (start 90.3265 90.71) (end 91.29 90.71) (width 0.2) (layer "F.Cu") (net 1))
 (segment (start 88.5 90.75) (end 90.2865 90.75) (width 0.2) (layer "F.Cu") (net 1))
 (segment (start 87.75 90) (end 88.5 90.75) (width 0.2) (layer "F.Cu") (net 1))
 (segment (start 87 90) (end 87.75 90) (width 0.2) (layer "F.Cu") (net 1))
 (segment (start 95.75 89) (end 96.124 89.374) (width 0.2) (layer "F.Cu") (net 1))
 (segment (start 90.2865 90.75) (end 90.3265 90.71) (width 0.2) (layer "F.Cu") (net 1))
 (segment (start 96.1135 91.944) (end 96.1135 90.0495) (width 0.2) (layer "F.Cu") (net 1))
 (segment (start 88.5 88.25) (end 117.475 88.25) (width 0.7) (layer "B.Cu") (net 1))
 (segment (start 126.703 90) (end 127.943 90) (width 0.7) (layer "B.Cu") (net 1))
 (segment (start 87 90) (end 84.5 90) (width 0.7) (layer "B.Cu") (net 1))
 (segment (start 117.7925 88.5675) (end 125.2705 88.5675) (width 0.7) (layer "B.Cu") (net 1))
 (segment (start 87 89.75) (end 88.5 88.25) (width 0.7) (layer "B.Cu") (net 1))
 (segment (start 117.475 88.25) (end 117.7925 88.5675) (width 0.7) (layer "B.Cu") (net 1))
 (segment (start 87 90) (end 87 89.75) (width 0.7) (layer "B.Cu") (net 1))
 (segment (start 125.2705 88.5675) (end 126.703 90) (width 0.7) (layer "B.Cu") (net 1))
 (segment (start 90.678 91.567) (end 90.678 92.2585) (width 0.2) (layer "F.Cu") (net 2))
 (segment (start 96.6635 90.805) (end 97.3815 90.087) (width 0.2) (layer "F.Cu") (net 2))
 (segment (start 94.024 90.039) (end 94.9245 90.039) (width 0.2) (layer "F.Cu") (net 2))
 (segment (start 94.9245 90.039) (end 95.5635 90.678) (width 0.2) (layer "F.Cu") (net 2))
 (segment (start 97.3815 90.087) (end 98.7375 90.087) (width 0.2) (layer "F.Cu") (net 2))
 (segment (start 92.841 90.039) (end 92.202 90.678) (width 0.2) (layer "F.Cu") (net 2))
 (segment (start 90.678 92.2585) (end 90.3265 92.61) (width 0.2) (layer "F.Cu") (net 2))
 (segment (start 94.024 90.039) (end 92.841 90.039) (width 0.2) (layer "F.Cu") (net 2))
 (via (at 95.5635 90.678) (size 0.5) (drill 0.3) (layers "F.Cu" "B.Cu") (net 2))
 (via (at 90.678 91.567) (size 0.5) (drill 0.3) (layers "F.Cu" "B.Cu") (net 2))
 (via (at 96.6635 90.805) (size 0.5) (drill 0.3) (layers "F.Cu" "B.Cu") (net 2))
 (via (at 92.202 90.678) (size 0.5) (drill 0.3) (layers "F.Cu" "B.Cu") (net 2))
 (segment (start 91.567 90.678) (end 90.678 91.567) (width 0.2) (layer "B.Cu") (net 2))
 (segment (start 92.202 90.678) (end 91.567 90.678) (width 0.2) (layer "B.Cu") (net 2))
 (segment (start 95.5635 90.678) (end 96.5365 90.678) (width 0.2) (layer "B.Cu") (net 2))
 (segment (start 96.5365 90.678) (end 96.6635 90.805) (width 0.2) (layer "B.Cu") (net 2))
 (segment (start 94.024 97.349) (end 94.175 97.5) (width 0.2) (layer "F.Cu") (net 8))
 (segment (start 90.3265 96.547) (end 90.578 96.547) (width 0.2) (layer "F.Cu") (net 8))
 (segment (start 94.024 95.5) (end 94.024 97.349) (width 0.2) (layer "F.Cu") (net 8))
 (segment (start 91.531 97.5) (end 94.175 97.5) (width 0.2) (layer "F.Cu") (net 8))
 (segment (start 90.578 96.547) (end 91.531 97.5) (width 0.2) (layer "F.Cu") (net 8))
 (segment (start 90.3265 94.647) (end 89.3645 94.647) (width 0.2) (layer "F.Cu") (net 7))
 (segment (start 96.1135 93.595) (end 96.1135 95.4895) (width 0.2) (layer "F.Cu") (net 7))
 (segment (start 90.3265 95.100052) (end 90.3265 94.647) (width 0.2) (layer "F.Cu") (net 7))
 (segment (start 96.1135 95.4895) (end 96.124 95.5) (width 0.2) (layer "F.Cu") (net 7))
 (segment (start 87.0115 97) (end 87 97) (width 0.2) (layer "F.Cu") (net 7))
 (segment (start 93.239 95.229) (end 93.239 95.937552) (width 0.2) (layer "F.Cu") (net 7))
 (segment (start 94.721 94.975) (end 93.493 94.975) (width 0.2) (layer "F.Cu") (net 7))
 (segment (start 91.423448 96.197) (end 90.3265 95.100052) (width 0.2) (layer "F.Cu") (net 7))
 (segment (start 93.493 94.975) (end 93.239 95.229) (width 0.2) (layer "F.Cu") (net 7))
 (segment (start 96.124 95.5) (end 95.246 95.5) (width 0.2) (layer "F.Cu") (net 7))
 (segment (start 93.239 95.937552) (end 92.979552 96.197) (width 0.2) (layer "F.Cu") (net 7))
 (segment (start 92.979552 96.197) (end 91.423448 96.197) (width 0.2) (layer "F.Cu") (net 7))
 (segment (start 95.246 95.5) (end 94.721 94.975) (width 0.2) (layer "F.Cu") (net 7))
 (segment (start 89.3645 94.647) (end 87.0115 97) (width 0.2) (layer "F.Cu") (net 7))
 (segment (start 84.5 97) (end 87 97) (width 0.7) (layer "B.Cu") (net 7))
 (segment (start 89 99) (end 87 97) (width 0.7) (layer "B.Cu") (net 7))
 (segment (start 127.943 97) (end 127.0755 97) (width 0.7) (layer "B.Cu") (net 7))
 (segment (start 125.0755 99) (end 89 99) (width 0.7) (layer "B.Cu") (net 7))
 (segment (start 127.0755 97) (end 125.0755 99) (width 0.7) (layer "B.Cu") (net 7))
 (segment (start 92.000776 94.943224) (end 92.2015 95.143948) (width 0.2) (layer "F.Cu") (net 3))
 (segment (start 92.837 94.488) (end 92.329 94.996) (width 0.2) (layer "F.Cu") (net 3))
 (segment (start 94.2885 93.6715) (end 93.472 94.488) (width 0.2) (layer "F.Cu") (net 3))
 (segment (start 90.557552 93.5) (end 92.000776 94.943224) (width 0.2) (layer "F.Cu") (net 3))
 (segment (start 92.329 94.996) (end 92.2015 95.1235) (width 0.2) (layer "F.Cu") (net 3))
 (segment (start 92.053552 94.996) (end 92.000776 94.943224) (width 0.2) (layer "F.Cu") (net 3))
 (segment (start 94.0045 91.66) (end 94.2885 91.944) (width 0.2) (layer "F.Cu") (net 3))
 (segment (start 94.2885 93.595) (end 94.2885 93.6715) (width 0.2) (layer "F.Cu") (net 3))
 (segment (start 87 93.5) (end 90.557552 93.5) (width 0.2) (layer "F.Cu") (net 3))
 (segment (start 94.2885 91.944) (end 94.2885 93.595) (width 0.2) (layer "F.Cu") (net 3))
 (segment (start 92.2015 95.1235) (end 92.2015 95.597) (width 0.2) (layer "F.Cu") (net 3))
 (segment (start 92.2015 95.143948) (end 92.2015 95.597) (width 0.2) (layer "F.Cu") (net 3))
 (segment (start 92.329 94.996) (end 92.053552 94.996) (width 0.2) (layer "F.Cu") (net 3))
 (segment (start 92.2015 91.66) (end 94.0045 91.66) (width 0.2) (layer "F.Cu") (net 3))
 (segment (start 93.472 94.488) (end 92.837 94.488) (width 0.2) (layer "F.Cu") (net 3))
 (segment (start 115.864 97.75) (end 90 97.75) (width 0.7) (layer "B.Cu") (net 3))
 (segment (start 127.943 93.5) (end 127.2035 93.5) (width 0.7) (layer "B.Cu") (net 3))
 (segment (start 90 97.75) (end 88.75 96.5) (width 0.7) (layer "B.Cu") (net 3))
 (segment (start 84.5 93.5) (end 87 93.5) (width 0.7) (layer "B.Cu") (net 3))
 (segment (start 88.75 96.5) (end 88.75 95.25) (width 0.7) (layer "B.Cu") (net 3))
 (segment (start 88.75 95.25) (end 87 93.5) (width 0.7) (layer "B.Cu") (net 3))
 (segment (start 125.736 94.9675) (end 118.6465 94.9675) (width 0.7) (layer "B.Cu") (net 3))
 (segment (start 118.6465 94.9675) (end 115.864 97.75) (width 0.7) (layer "B.Cu") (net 3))
 (segment (start 127.2035 93.5) (end 125.736 94.9675) (width 0.7) (layer "B.Cu") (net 3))
 (segment (start 115.25 87.65) (end 103.35 87.65) (width 0.7) (layer "F.Cu") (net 4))
 (segment (start 117.6175 90.0175) (end 115.25 87.65) (width 0.7) (layer "F.Cu") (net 4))
 (segment (start 101.9375 90.087) (end 101.9375 97.087) (width 0.7) (layer "F.Cu") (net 4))
 (segment (start 120.3575 90.0175) (end 117.6175 90.0175) (width 0.7) (layer "F.Cu") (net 4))
 (segment (start 101.9375 89.0625) (end 101.9375 90.087) (width 0.7) (layer "F.Cu") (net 4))
 (segment (start 103.35 87.65) (end 101.9375 89.0625) (width 0.7) (layer "F.Cu") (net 4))
 (segment (start 110.25 97.5) (end 116.2675 97.5) (width 0.7) (layer "F.Cu") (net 6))
 (segment (start 106.3375 97.087) (end 106.3375 90.087) (width 0.7) (layer "F.Cu") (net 6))
 (segment (start 109.837 97.087) (end 110.25 97.5) (width 0.7) (layer "F.Cu") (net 6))
 (segment (start 106.3375 97.087) (end 109.837 97.087) (width 0.7) (layer "F.Cu") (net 6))
 (segment (start 116.75 97.0175) (end 120.3575 97.0175) (width 0.7) (layer "F.Cu") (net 6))
 (segment (start 116.2675 97.5) (end 116.75 97.0175) (width 0.7) (layer "F.Cu") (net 6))
 (segment (start 104.1375 90.087) (end 105.6745 88.55) (width 0.7) (layer "F.Cu") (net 5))
 (segment (start 104.1375 97.087) (end 104.1375 90.087) (width 0.7) (layer "F.Cu") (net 5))
 (segment (start 114.331 88.55) (end 119.2985 93.5175) (width 0.7) (layer "F.Cu") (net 5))
 (segment (start 119.2985 93.5175) (end 120.3575 93.5175) (width 0.7) (layer "F.Cu") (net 5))
 (segment (start 105.6745 88.55) (end 114.331 88.55) (width 0.7) (layer "F.Cu") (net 5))
 (segment (start 98.3245 97.5) (end 98.7375 97.087) (width 0.2) (layer "F.Cu") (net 9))
 (segment (start 96 97.5) (end 98.3245 97.5) (width 0.2) (layer "F.Cu") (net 9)))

